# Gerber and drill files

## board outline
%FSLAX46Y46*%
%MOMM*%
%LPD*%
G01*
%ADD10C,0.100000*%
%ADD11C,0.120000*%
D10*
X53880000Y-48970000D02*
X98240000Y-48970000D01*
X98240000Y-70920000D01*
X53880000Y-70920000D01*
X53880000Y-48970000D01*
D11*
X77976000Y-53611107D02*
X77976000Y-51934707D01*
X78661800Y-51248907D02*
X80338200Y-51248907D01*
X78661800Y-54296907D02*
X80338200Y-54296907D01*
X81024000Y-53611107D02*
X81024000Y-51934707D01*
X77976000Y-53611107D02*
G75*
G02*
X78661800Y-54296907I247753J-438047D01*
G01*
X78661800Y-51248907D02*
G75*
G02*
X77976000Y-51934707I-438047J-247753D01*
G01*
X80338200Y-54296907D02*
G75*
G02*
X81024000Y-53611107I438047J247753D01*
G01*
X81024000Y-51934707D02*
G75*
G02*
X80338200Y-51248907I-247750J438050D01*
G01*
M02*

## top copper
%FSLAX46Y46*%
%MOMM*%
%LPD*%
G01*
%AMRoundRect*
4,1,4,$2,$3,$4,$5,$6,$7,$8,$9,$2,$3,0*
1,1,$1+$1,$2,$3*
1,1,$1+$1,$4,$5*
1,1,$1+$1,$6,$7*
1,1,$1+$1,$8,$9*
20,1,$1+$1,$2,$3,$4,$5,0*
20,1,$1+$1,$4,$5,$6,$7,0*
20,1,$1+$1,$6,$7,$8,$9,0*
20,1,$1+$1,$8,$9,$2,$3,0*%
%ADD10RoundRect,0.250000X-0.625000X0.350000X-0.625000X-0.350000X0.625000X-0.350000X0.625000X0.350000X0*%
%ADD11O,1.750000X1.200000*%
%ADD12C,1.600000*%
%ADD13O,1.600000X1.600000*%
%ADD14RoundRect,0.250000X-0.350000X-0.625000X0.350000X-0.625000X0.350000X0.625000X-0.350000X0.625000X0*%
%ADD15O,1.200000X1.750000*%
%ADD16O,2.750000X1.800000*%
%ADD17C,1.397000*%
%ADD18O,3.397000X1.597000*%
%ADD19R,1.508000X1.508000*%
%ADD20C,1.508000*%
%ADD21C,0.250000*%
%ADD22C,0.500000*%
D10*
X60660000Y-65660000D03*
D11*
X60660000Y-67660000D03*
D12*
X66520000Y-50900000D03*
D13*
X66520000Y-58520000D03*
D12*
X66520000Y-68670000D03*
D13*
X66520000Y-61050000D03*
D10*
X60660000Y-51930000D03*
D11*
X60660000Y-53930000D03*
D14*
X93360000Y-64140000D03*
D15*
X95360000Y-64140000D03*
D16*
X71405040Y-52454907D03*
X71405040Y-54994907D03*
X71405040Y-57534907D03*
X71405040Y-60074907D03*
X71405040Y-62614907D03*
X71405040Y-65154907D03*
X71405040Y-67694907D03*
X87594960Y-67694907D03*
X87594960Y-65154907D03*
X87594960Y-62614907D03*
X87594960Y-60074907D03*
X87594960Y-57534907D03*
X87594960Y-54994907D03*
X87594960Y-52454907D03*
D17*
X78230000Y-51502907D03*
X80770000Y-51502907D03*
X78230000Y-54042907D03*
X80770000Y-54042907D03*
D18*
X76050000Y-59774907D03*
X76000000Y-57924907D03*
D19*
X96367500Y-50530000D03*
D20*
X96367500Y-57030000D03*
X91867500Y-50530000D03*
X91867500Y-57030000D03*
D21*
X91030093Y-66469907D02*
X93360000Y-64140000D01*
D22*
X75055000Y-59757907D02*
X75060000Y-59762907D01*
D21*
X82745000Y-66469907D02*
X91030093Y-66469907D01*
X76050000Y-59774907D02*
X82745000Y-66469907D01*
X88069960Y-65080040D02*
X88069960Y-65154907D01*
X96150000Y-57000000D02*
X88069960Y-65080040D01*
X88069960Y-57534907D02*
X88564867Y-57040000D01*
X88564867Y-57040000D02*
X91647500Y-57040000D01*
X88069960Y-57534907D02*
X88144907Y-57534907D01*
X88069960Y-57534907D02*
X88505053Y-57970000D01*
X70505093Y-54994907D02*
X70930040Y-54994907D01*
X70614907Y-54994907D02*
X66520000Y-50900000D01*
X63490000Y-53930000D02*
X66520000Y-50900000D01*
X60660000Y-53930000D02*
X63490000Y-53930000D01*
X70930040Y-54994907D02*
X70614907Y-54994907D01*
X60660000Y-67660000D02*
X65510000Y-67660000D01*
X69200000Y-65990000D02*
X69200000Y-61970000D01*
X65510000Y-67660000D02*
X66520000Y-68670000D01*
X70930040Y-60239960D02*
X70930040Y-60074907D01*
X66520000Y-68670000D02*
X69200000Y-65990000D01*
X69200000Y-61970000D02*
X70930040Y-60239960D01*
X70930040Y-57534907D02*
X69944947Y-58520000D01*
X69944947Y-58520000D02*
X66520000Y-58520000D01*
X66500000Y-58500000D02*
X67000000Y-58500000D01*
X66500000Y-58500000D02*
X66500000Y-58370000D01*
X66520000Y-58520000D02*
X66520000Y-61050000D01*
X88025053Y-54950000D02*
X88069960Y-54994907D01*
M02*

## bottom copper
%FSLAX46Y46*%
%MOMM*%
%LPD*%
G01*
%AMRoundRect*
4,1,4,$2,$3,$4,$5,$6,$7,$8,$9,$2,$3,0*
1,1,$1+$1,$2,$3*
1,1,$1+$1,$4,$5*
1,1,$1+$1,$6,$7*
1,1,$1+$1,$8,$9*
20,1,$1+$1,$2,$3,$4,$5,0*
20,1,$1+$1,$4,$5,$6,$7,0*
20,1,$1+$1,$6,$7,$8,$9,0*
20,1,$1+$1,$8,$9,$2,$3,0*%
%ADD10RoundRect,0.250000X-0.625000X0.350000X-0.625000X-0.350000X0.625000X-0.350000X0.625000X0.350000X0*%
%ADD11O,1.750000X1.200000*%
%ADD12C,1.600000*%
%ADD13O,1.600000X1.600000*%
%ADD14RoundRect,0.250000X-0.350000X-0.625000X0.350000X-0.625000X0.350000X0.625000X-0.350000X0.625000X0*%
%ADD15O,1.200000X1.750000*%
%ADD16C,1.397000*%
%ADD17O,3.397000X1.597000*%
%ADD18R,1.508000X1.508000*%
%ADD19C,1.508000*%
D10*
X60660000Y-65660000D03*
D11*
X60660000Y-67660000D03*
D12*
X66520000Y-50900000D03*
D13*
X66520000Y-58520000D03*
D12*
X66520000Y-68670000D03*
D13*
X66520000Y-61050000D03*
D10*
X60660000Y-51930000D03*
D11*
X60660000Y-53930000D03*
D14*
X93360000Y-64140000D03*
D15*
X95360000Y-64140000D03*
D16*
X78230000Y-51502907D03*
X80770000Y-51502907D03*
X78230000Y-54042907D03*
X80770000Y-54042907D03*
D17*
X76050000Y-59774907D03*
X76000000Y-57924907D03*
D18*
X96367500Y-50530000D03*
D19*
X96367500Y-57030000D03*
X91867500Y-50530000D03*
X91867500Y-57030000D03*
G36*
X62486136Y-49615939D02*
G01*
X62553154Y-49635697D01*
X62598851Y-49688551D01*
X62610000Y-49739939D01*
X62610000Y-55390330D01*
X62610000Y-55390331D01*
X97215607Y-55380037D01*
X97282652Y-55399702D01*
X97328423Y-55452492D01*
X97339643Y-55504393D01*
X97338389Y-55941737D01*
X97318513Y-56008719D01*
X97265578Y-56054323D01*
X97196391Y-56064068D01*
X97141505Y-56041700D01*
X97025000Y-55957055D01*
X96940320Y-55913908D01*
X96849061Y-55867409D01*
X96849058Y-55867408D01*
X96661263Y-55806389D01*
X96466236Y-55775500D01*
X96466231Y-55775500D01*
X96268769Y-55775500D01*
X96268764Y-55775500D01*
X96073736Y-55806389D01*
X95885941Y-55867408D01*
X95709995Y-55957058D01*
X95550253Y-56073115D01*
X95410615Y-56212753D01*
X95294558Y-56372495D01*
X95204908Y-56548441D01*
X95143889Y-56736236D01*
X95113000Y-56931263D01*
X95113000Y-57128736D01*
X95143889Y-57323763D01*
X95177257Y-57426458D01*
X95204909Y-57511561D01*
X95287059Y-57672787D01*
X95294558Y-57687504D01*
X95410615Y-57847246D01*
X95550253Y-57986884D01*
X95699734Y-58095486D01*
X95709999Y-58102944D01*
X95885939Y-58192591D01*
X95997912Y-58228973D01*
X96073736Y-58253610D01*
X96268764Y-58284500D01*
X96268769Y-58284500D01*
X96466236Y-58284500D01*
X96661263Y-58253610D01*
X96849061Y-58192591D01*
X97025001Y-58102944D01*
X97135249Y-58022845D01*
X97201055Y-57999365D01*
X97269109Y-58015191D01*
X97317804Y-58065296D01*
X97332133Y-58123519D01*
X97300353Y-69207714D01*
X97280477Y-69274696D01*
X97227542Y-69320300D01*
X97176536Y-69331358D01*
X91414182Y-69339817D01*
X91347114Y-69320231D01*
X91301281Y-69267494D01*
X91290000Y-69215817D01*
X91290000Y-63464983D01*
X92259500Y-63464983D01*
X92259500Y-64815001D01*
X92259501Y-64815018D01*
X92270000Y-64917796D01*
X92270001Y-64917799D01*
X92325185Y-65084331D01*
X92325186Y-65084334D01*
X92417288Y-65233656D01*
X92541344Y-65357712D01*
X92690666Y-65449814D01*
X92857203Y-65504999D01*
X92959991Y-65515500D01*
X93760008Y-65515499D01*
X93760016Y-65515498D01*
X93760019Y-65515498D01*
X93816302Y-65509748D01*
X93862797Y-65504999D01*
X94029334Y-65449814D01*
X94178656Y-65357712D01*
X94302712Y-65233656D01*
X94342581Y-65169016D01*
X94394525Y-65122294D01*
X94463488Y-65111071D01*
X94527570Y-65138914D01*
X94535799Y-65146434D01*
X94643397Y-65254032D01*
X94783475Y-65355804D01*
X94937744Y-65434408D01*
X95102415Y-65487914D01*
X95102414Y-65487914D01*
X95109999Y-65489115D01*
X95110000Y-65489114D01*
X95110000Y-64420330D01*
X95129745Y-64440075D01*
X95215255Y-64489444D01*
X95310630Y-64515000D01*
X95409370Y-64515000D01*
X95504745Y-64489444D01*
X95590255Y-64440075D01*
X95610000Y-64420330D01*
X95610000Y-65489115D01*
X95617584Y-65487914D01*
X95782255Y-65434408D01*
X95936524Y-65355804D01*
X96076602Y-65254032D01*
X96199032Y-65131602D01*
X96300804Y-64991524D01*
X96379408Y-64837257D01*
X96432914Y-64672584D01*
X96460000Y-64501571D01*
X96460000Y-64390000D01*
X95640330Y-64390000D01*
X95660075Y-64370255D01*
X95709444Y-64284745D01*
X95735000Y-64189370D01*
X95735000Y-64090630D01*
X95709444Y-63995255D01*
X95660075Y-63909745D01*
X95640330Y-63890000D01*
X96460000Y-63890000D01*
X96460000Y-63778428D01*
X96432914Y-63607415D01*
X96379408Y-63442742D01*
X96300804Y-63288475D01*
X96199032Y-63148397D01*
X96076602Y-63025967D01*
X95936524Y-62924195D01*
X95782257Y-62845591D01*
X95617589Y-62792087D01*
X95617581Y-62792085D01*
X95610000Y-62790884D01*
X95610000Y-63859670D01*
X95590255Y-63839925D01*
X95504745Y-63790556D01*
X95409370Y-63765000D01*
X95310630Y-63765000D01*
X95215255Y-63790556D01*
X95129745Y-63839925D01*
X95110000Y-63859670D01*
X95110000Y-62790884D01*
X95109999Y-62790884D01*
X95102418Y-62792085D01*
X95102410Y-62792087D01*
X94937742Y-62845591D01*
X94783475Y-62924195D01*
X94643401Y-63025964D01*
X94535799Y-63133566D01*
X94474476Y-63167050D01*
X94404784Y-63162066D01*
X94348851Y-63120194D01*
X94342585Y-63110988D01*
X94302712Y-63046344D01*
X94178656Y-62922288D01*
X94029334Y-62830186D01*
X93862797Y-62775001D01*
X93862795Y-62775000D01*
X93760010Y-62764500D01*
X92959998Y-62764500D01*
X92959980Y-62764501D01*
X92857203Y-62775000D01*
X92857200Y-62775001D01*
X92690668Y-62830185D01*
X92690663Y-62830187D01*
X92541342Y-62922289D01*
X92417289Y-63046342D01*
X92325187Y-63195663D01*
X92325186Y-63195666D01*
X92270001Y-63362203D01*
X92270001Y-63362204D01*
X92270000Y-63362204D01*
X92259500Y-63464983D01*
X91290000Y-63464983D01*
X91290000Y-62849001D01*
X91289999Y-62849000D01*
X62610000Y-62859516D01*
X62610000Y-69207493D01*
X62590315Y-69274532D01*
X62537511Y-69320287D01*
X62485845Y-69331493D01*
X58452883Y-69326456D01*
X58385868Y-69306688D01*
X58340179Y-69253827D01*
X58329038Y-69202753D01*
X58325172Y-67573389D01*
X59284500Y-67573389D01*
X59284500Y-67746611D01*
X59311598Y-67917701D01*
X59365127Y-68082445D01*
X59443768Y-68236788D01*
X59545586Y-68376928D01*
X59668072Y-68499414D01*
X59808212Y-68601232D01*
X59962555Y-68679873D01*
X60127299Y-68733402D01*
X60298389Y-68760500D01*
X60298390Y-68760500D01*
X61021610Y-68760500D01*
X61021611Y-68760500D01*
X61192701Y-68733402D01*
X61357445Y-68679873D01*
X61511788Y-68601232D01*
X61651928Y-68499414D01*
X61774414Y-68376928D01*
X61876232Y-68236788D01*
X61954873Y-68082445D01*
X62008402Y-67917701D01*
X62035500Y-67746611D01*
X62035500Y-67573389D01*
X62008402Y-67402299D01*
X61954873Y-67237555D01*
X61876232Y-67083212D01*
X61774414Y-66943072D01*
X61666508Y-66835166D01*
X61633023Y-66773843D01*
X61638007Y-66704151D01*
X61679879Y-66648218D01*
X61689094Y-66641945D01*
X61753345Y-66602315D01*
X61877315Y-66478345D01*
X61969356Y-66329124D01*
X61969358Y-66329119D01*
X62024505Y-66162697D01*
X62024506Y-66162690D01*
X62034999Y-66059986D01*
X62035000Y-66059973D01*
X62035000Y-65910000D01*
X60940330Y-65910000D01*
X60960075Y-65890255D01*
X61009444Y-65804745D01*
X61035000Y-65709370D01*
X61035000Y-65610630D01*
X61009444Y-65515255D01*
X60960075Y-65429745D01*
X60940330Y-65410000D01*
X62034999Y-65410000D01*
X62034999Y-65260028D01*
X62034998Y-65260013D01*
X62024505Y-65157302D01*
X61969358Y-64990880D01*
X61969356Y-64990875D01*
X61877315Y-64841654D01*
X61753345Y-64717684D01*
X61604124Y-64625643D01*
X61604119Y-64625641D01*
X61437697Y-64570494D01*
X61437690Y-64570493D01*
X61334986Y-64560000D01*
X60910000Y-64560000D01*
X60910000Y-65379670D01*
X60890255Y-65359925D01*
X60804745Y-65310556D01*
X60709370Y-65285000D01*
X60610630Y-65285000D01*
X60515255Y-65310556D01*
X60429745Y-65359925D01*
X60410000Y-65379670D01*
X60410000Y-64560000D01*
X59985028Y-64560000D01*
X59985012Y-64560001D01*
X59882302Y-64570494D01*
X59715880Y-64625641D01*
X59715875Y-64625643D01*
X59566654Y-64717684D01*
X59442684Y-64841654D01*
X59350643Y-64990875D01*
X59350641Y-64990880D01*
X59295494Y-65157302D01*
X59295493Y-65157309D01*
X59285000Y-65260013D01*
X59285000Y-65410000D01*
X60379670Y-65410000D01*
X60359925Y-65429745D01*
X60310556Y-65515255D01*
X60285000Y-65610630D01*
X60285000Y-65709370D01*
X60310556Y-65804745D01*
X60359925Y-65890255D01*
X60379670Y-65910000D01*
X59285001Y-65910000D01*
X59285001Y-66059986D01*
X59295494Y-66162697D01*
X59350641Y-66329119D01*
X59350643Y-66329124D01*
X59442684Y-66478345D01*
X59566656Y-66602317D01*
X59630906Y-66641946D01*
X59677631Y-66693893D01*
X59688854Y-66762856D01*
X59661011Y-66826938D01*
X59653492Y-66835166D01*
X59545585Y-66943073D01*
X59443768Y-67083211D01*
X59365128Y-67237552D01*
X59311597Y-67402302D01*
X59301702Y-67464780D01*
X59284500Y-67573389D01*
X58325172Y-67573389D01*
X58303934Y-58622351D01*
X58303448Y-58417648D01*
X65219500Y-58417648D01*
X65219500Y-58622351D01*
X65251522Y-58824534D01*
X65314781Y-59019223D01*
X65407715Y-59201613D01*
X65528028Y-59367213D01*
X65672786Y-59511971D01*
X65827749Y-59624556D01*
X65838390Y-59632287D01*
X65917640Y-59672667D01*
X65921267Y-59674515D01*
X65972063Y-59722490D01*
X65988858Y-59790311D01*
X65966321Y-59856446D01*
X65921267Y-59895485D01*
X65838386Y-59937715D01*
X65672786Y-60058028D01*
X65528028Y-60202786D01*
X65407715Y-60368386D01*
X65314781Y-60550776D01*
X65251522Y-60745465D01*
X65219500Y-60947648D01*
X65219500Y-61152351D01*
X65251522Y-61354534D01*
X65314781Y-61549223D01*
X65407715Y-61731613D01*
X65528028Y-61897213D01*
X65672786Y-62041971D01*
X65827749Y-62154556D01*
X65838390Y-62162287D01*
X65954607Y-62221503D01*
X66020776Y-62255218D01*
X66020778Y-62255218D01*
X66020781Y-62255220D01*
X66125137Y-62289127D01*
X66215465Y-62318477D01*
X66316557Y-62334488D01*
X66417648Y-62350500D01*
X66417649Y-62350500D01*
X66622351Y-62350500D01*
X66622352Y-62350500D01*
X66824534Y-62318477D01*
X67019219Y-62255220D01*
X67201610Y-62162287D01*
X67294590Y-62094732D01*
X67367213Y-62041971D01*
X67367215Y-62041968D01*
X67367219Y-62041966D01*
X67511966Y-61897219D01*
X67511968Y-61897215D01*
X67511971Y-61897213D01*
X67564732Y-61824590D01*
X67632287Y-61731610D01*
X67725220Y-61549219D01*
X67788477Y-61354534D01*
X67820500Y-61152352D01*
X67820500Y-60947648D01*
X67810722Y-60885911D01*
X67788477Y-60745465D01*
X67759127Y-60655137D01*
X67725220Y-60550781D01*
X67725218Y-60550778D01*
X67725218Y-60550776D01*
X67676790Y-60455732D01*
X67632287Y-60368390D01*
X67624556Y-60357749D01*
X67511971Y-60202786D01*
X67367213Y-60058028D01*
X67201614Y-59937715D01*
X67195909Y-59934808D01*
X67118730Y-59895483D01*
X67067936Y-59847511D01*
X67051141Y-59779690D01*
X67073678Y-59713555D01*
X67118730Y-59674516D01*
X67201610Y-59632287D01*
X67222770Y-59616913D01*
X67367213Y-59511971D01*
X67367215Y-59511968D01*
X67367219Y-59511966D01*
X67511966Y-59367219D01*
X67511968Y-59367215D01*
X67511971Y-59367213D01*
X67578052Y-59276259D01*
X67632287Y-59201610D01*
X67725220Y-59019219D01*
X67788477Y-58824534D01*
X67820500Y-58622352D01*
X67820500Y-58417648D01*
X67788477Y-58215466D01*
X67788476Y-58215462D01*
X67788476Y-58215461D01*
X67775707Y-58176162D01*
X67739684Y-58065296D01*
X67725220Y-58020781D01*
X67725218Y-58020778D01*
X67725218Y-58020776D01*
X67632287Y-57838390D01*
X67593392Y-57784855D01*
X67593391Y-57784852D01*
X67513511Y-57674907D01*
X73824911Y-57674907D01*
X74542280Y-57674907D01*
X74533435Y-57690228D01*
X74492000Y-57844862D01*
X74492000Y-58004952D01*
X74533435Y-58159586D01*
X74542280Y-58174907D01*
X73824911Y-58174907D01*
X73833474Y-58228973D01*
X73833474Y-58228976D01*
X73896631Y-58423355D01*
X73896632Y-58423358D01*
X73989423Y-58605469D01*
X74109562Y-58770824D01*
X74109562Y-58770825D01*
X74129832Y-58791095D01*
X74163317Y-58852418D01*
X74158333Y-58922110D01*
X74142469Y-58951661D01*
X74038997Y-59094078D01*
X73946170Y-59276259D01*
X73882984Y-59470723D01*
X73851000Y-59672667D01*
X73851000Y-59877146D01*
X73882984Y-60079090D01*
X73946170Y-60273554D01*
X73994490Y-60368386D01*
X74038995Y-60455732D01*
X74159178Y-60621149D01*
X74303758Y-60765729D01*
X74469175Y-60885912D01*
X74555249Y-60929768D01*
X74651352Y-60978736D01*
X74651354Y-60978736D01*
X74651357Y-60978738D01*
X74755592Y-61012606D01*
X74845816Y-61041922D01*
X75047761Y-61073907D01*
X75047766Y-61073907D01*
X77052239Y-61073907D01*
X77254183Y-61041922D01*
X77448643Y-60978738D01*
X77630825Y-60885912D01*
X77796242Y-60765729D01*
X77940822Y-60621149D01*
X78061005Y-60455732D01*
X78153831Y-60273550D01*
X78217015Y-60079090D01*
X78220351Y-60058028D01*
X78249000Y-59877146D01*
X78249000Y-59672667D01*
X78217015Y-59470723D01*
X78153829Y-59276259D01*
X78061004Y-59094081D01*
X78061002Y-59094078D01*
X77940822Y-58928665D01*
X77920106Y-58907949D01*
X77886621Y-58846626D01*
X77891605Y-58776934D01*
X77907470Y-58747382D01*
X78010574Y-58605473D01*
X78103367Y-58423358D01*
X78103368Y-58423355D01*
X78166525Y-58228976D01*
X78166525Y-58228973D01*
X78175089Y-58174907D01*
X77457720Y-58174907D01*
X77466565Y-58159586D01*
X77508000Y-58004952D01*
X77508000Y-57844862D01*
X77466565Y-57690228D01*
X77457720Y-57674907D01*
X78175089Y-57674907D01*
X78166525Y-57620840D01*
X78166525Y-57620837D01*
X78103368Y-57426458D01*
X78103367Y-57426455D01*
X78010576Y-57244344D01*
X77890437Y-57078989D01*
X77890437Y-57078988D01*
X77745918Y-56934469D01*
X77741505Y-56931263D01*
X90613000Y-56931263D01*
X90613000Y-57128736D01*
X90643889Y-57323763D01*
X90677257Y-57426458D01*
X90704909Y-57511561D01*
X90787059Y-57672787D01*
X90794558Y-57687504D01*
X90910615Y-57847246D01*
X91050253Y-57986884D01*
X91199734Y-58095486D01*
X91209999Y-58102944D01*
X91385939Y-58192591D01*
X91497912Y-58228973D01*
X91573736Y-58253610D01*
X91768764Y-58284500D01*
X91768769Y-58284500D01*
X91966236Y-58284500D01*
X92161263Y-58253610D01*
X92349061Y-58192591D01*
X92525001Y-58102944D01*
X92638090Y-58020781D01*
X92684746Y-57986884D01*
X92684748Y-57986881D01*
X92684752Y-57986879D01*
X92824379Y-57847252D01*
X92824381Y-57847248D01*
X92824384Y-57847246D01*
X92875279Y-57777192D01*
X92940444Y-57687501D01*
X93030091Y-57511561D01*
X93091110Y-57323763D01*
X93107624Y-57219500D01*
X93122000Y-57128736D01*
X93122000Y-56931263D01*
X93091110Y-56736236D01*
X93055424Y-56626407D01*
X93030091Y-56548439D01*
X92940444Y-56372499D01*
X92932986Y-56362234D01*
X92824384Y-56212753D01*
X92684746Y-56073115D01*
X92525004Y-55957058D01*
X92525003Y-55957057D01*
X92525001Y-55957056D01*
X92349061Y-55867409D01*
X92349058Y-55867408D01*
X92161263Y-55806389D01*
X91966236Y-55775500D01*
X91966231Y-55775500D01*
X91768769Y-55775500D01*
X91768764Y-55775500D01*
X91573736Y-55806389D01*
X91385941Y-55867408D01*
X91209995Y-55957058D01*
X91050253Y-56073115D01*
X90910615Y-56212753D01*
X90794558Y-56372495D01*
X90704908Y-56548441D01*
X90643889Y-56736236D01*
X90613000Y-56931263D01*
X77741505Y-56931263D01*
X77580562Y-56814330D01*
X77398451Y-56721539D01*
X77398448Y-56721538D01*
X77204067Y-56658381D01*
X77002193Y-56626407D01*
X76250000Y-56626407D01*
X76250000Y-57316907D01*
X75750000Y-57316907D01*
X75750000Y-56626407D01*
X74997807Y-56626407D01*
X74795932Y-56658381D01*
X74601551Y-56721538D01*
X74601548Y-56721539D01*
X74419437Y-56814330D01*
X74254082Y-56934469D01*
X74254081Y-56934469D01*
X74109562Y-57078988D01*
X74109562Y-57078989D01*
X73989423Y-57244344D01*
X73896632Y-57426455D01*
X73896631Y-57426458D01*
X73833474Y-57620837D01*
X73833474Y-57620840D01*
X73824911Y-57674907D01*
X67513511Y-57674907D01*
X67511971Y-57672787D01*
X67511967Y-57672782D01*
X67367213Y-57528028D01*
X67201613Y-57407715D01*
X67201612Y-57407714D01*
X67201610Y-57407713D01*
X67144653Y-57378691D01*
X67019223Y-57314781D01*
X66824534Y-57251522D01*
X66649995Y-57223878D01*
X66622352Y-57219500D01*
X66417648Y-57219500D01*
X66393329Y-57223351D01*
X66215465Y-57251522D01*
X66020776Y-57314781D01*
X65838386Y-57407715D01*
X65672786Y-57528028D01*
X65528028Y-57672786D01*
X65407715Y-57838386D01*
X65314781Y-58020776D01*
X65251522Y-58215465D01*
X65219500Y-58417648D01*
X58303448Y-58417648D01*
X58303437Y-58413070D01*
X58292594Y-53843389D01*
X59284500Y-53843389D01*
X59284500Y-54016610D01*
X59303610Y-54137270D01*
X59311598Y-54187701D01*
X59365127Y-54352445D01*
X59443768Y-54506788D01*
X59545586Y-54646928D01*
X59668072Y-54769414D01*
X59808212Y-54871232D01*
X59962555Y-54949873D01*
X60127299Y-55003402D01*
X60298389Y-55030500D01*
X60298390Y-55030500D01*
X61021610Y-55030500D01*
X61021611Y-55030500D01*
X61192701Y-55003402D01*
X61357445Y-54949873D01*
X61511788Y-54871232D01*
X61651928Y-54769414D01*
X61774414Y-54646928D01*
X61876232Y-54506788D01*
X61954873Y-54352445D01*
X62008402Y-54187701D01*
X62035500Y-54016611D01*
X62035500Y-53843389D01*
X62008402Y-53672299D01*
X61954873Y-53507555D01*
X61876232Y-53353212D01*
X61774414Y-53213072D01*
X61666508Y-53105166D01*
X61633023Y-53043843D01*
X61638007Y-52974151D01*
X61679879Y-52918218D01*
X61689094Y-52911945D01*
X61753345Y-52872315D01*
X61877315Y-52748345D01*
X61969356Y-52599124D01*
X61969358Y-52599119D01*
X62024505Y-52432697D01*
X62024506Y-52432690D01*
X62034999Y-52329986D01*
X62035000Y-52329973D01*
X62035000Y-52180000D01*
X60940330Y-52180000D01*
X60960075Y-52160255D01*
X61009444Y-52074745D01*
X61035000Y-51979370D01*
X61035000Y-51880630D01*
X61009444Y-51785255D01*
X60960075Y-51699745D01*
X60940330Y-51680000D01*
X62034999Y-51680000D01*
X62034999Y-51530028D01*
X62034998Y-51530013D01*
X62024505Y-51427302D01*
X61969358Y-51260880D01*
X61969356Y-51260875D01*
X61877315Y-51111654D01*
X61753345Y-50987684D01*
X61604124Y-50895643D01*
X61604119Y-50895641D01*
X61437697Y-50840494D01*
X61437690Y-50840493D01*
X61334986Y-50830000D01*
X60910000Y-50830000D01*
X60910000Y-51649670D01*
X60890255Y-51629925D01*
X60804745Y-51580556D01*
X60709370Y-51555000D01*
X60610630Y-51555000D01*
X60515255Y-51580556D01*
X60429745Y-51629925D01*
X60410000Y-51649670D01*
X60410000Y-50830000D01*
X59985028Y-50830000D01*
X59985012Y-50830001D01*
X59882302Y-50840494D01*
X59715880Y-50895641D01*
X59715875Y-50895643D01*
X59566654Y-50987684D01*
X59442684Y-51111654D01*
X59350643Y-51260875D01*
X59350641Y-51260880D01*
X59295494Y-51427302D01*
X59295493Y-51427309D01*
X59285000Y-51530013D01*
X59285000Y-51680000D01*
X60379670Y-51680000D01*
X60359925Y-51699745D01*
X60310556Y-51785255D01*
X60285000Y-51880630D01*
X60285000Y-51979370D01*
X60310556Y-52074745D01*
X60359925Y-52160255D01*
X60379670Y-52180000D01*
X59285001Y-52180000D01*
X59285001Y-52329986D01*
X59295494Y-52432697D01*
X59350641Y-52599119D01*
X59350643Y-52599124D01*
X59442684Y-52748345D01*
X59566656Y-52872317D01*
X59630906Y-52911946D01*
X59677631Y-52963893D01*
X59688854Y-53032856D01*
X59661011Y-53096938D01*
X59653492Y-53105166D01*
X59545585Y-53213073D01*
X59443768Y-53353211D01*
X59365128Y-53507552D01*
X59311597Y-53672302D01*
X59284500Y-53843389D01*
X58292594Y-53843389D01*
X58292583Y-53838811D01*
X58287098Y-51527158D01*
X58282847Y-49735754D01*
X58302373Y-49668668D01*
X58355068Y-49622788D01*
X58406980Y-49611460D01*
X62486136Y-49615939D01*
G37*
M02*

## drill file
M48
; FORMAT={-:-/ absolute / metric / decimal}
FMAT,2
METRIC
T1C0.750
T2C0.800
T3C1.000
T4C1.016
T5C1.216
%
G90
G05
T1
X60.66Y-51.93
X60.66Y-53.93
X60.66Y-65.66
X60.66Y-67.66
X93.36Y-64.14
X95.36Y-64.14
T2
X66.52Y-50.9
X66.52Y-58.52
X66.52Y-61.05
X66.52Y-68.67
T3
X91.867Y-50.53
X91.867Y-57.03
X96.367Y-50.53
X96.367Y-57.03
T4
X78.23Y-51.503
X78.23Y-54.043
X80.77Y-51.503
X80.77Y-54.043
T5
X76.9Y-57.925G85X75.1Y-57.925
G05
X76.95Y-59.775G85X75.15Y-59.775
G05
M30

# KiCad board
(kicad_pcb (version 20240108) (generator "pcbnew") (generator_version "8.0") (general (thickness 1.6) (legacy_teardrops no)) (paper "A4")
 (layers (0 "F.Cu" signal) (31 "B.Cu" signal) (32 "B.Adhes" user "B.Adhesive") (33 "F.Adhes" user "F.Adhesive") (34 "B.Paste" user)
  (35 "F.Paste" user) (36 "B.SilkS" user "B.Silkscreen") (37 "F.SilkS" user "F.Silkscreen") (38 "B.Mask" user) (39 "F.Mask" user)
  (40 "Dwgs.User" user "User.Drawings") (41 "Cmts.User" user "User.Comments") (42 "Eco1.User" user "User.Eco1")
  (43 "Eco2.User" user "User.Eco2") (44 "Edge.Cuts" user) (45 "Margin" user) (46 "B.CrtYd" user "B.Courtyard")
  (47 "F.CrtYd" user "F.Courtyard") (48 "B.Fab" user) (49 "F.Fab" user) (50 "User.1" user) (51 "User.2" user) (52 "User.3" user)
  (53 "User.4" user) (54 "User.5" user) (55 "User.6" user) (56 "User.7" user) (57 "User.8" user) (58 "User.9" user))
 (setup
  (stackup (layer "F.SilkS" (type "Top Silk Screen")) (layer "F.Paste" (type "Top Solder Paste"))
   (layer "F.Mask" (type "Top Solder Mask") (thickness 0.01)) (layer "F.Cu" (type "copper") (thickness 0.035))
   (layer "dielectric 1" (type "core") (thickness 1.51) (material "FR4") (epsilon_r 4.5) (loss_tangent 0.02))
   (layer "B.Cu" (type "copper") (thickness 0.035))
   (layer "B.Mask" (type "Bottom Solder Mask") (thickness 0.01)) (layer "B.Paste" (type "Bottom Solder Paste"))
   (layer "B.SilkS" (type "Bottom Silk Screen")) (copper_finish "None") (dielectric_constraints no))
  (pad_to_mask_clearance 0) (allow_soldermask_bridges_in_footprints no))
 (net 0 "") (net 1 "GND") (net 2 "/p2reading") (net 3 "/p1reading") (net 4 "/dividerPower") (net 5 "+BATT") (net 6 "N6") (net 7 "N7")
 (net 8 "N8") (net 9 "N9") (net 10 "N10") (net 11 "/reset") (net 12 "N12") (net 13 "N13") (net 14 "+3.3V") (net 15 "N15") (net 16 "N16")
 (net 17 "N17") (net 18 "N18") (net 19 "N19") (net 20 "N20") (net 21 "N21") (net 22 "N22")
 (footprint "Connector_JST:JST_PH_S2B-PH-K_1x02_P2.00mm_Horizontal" (layer "F.Cu") (at 60.66 65.66 -90)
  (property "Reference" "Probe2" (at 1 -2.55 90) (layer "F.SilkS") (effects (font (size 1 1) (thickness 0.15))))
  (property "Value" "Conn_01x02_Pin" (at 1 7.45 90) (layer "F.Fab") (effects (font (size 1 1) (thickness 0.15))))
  (pad "1" thru_hole roundrect (at 0 0 270) (size 1.2 1.75) (drill 0.75) (layers "*.Cu" "*.Mask") (remove_unused_layers no)
   (roundrect_rratio 0.208333) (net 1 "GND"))
  (pad "2" thru_hole oval (at 2 0 270) (size 1.2 1.75) (drill 0.75) (layers "*.Cu" "*.Mask") (remove_unused_layers no) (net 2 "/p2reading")))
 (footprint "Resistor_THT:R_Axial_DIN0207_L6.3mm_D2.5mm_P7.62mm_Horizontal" (layer "F.Cu") (at 66.52 50.9 -90)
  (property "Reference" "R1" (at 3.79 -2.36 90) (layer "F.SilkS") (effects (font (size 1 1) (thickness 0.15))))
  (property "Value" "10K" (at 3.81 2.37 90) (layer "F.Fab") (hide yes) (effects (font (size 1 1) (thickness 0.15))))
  (pad "1" thru_hole circle (at 0 0 270) (size 1.6 1.6) (drill 0.8) (layers "*.Cu" "*.Mask") (remove_unused_layers no) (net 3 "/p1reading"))
  (pad "2" thru_hole oval (at 7.62 0 270) (size 1.6 1.6) (drill 0.8) (layers "*.Cu" "*.Mask") (remove_unused_layers no)
   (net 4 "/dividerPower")))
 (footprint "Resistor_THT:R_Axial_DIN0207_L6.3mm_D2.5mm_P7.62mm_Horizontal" (layer "F.Cu") (at 66.52 68.67 90)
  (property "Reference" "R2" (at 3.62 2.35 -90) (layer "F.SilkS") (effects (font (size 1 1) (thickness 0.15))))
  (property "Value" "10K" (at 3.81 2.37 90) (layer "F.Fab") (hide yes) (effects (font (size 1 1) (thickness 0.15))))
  (pad "1" thru_hole circle (at 0 0 90) (size 1.6 1.6) (drill 0.8) (layers "*.Cu" "*.Mask") (remove_unused_layers no) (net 2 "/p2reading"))
  (pad "2" thru_hole oval (at 7.62 0 90) (size 1.6 1.6) (drill 0.8) (layers "*.Cu" "*.Mask") (remove_unused_layers no)
   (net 4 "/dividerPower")))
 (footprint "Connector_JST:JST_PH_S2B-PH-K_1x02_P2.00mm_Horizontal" (layer "F.Cu") (at 60.66 51.93 -90)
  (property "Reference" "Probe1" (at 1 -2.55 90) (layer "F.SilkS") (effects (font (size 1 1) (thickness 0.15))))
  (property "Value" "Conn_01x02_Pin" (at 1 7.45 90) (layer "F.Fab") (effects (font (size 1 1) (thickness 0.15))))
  (pad "1" thru_hole roundrect (at 0 0 270) (size 1.2 1.75) (drill 0.75) (layers "*.Cu" "*.Mask") (remove_unused_layers no)
   (roundrect_rratio 0.208333) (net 1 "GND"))
  (pad "2" thru_hole oval (at 2 0 270) (size 1.2 1.75) (drill 0.75) (layers "*.Cu" "*.Mask") (remove_unused_layers no) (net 3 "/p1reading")))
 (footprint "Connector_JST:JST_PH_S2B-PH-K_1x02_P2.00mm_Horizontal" (layer "F.Cu") (at 93.36 64.14)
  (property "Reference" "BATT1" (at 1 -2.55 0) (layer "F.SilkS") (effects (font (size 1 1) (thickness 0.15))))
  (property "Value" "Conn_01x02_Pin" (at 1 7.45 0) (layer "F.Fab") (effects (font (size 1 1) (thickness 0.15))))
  (pad "1" thru_hole roundrect (at 0 0) (size 1.2 1.75) (drill 0.75) (layers "*.Cu" "*.Mask") (remove_unused_layers no)
   (roundrect_rratio 0.208333) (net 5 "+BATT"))
  (pad "2" thru_hole oval (at 2 0) (size 1.2 1.75) (drill 0.75) (layers "*.Cu" "*.Mask") (remove_unused_layers no) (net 1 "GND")))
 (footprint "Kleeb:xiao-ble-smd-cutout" (layer "F.Cu") (at 79.5 60.074907)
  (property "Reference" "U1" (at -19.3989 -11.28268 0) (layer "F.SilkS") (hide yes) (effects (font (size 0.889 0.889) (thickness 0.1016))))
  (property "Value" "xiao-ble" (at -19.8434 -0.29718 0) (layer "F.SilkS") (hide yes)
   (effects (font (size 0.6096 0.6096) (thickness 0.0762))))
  (fp_line (start -1.524 -6.4638) (end -1.524 -8.1402) (stroke (width 0.12) (type solid)) (layer "Edge.Cuts"))
  (fp_line (start -0.8382 -8.826) (end 0.8382 -8.826) (stroke (width 0.12) (type solid)) (layer "Edge.Cuts"))
  (fp_line (start -0.8382 -5.778) (end 0.8382 -5.778) (stroke (width 0.12) (type solid)) (layer "Edge.Cuts"))
  (fp_line (start 1.524 -6.4638) (end 1.524 -8.1402) (stroke (width 0.12) (type solid)) (layer "Edge.Cuts"))
  (fp_arc (start -1.524 -6.4638) (mid -0.920391 -6.381609) (end -0.8382 -5.778) (stroke (width 0.12) (type solid)) (layer "Edge.Cuts"))
  (fp_arc (start -0.8382 -8.826) (mid -0.920391 -8.222391) (end -1.524 -8.1402) (stroke (width 0.12) (type solid)) (layer "Edge.Cuts"))
  (fp_arc (start 0.8382 -5.778) (mid 0.920391 -6.381609) (end 1.524 -6.4638) (stroke (width 0.12) (type solid)) (layer "Edge.Cuts"))
  (fp_arc (start 1.524 -8.1402) (mid 0.920393 -8.222393) (end 0.8382 -8.826) (stroke (width 0.12) (type solid)) (layer "Edge.Cuts"))
  (pad "1" smd oval (at -8.56996 -7.62 180) (size 2.75 1.8) (drill (offset -0.475 0)) (layers "F.Cu" "F.Paste" "F.Mask") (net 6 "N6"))
  (pad "2" smd oval (at -8.56996 -5.08 180) (size 2.75 1.8) (drill (offset -0.475 0)) (layers "F.Cu" "F.Paste" "F.Mask")
   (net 3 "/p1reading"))
  (pad "3" smd oval (at -8.56996 -2.54 180) (size 2.75 1.8) (drill (offset -0.475 0)) (layers "F.Cu" "F.Paste" "F.Mask")
   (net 4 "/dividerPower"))
  (pad "4" smd oval (at -8.56996 0 180) (size 2.75 1.8) (drill (offset -0.475 0)) (layers "F.Cu" "F.Paste" "F.Mask") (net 2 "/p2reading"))
  (pad "5" smd oval (at -8.56996 2.54 180) (size 2.75 1.8) (drill (offset -0.475 0)) (layers "F.Cu" "F.Paste" "F.Mask") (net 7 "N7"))
  (pad "6" smd oval (at -8.56996 5.08 180) (size 2.75 1.8) (drill (offset -0.475 0)) (layers "F.Cu" "F.Paste" "F.Mask") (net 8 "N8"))
  (pad "7" smd oval (at -8.56996 7.62 180) (size 2.75 1.8) (drill (offset -0.475 0)) (layers "F.Cu" "F.Paste" "F.Mask") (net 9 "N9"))
  (pad "8" smd oval (at 8.56996 7.62) (size 2.75 1.8) (drill (offset -0.475 0)) (layers "F.Cu" "F.Paste" "F.Mask") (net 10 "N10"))
  (pad "9" smd oval (at 8.56996 5.08) (size 2.75 1.8) (drill (offset -0.475 0)) (layers "F.Cu" "F.Paste" "F.Mask") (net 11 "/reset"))
  (pad "10" smd oval (at 8.56996 2.54) (size 2.75 1.8) (drill (offset -0.475 0)) (layers "F.Cu" "F.Paste" "F.Mask") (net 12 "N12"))
  (pad "11" smd oval (at 8.56996 0) (size 2.75 1.8) (drill (offset -0.475 0)) (layers "F.Cu" "F.Paste" "F.Mask") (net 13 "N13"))
  (pad "12" smd oval (at 8.56996 -2.54) (size 2.75 1.8) (drill (offset -0.475 0)) (layers "F.Cu" "F.Paste" "F.Mask") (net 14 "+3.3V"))
  (pad "13" smd oval (at 8.56996 -5.08) (size 2.75 1.8) (drill (offset -0.475 0)) (layers "F.Cu" "F.Paste" "F.Mask") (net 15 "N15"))
  (pad "14" smd oval (at 8.56996 -7.62) (size 2.75 1.8) (drill (offset -0.475 0)) (layers "F.Cu" "F.Paste" "F.Mask") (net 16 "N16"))
  (pad "15" thru_hole circle (at -1.27 -8.572 90) (size 1.397 1.397) (drill 1.016) (layers "*.Cu" "*.Mask") (remove_unused_layers no)
   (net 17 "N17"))
  (pad "16" thru_hole circle (at 1.27 -8.572 90) (size 1.397 1.397) (drill 1.016) (layers "*.Cu" "*.Mask") (remove_unused_layers no)
   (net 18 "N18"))
  (pad "17" thru_hole circle (at -1.27 -6.032 90) (size 1.397 1.397) (drill 1.016) (layers "*.Cu" "*.Mask") (remove_unused_layers no)
   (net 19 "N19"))
  (pad "18" thru_hole circle (at 1.27 -6.032 90) (size 1.397 1.397) (drill 1.016) (layers "*.Cu" "*.Mask") (remove_unused_layers no)
   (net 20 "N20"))
  (pad "19" thru_hole oval (at -3.45 -0.3 180) (size 3.397 1.597) (drill oval 3.016 1.216) (layers "*.Cu" "*.Mask")
   (remove_unused_layers no) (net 5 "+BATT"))
  (pad "20" thru_hole oval (at -3.5 -2.15 180) (size 3.397 1.597) (drill oval 3.016 1.216) (layers "*.Cu" "*.Mask")
   (remove_unused_layers no) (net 1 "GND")))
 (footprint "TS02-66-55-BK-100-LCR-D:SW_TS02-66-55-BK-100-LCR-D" (layer "F.Cu") (at 94.1175 53.78 -90)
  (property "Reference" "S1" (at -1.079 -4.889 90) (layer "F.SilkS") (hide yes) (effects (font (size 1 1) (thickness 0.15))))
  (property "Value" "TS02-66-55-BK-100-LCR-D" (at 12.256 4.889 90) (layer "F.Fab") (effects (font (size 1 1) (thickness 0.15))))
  (pad "1" thru_hole rect (at -3.25 -2.25 270) (size 1.508 1.508) (drill 1) (layers "*.Cu" "*.Mask") (remove_unused_layers no)
   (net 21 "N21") (solder_mask_margin 0.102))
  (pad "2" thru_hole circle (at 3.25 -2.25 270) (size 1.508 1.508) (drill 1) (layers "*.Cu" "*.Mask") (remove_unused_layers no)
   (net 11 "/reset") (solder_mask_margin 0.102))
  (pad "3" thru_hole circle (at -3.25 2.25 270) (size 1.508 1.508) (drill 1) (layers "*.Cu" "*.Mask") (remove_unused_layers no)
   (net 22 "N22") (solder_mask_margin 0.102))
  (pad "4" thru_hole circle (at 3.25 2.25 270) (size 1.508 1.508) (drill 1) (layers "*.Cu" "*.Mask") (remove_unused_layers no)
   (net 14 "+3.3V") (solder_mask_margin 0.102)))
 (gr_rect (start 53.88 48.97) (end 98.24 70.92) (stroke (width 0.1) (type default)) (fill none) (layer "Edge.Cuts"))
 (segment (start 91.030093 66.469907) (end 93.36 64.14) (width 0.25) (layer "F.Cu") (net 5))
 (segment (start 75.055 59.757907) (end 75.06 59.762907) (width 0.5) (layer "F.Cu") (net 5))
 (segment (start 82.745 66.469907) (end 91.030093 66.469907) (width 0.25) (layer "F.Cu") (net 5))
 (segment (start 76.05 59.774907) (end 82.745 66.469907) (width 0.25) (layer "F.Cu") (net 5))
 (segment (start 88.06996 65.08004) (end 88.06996 65.154907) (width 0.25) (layer "F.Cu") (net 11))
 (segment (start 96.15 57) (end 88.06996 65.08004) (width 0.25) (layer "F.Cu") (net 11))
 (segment (start 88.06996 57.534907) (end 88.564867 57.04) (width 0.25) (layer "F.Cu") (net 14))
 (segment (start 88.564867 57.04) (end 91.6475 57.04) (width 0.25) (layer "F.Cu") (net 14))
 (segment (start 88.06996 57.534907) (end 88.144907 57.534907) (width 0.25) (layer "F.Cu") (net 14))
 (segment (start 88.06996 57.534907) (end 88.505053 57.97) (width 0.25) (layer "F.Cu") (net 14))
 (segment (start 70.505093 54.994907) (end 70.93004 54.994907) (width 0.25) (layer "F.Cu") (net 3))
 (segment (start 70.614907 54.994907) (end 66.52 50.9) (width 0.25) (layer "F.Cu") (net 3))
 (segment (start 63.49 53.93) (end 66.52 50.9) (width 0.25) (layer "F.Cu") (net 3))
 (segment (start 60.66 53.93) (end 63.49 53.93) (width 0.25) (layer "F.Cu") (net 3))
 (segment (start 70.93004 54.994907) (end 70.614907 54.994907) (width 0.25) (layer "F.Cu") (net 3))
 (segment (start 60.66 67.66) (end 65.51 67.66) (width 0.25) (layer "F.Cu") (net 2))
 (segment (start 69.2 65.99) (end 69.2 61.97) (width 0.25) (layer "F.Cu") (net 2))
 (segment (start 65.51 67.66) (end 66.52 68.67) (width 0.25) (layer "F.Cu") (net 2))
 (segment (start 70.93004 60.23996) (end 70.93004 60.074907) (width 0.25) (layer "F.Cu") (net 2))
 (segment (start 66.52 68.67) (end 69.2 65.99) (width 0.25) (layer "F.Cu") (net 2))
 (segment (start 69.2 61.97) (end 70.93004 60.23996) (width 0.25) (layer "F.Cu") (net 2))
 (segment (start 70.93004 57.534907) (end 69.944947 58.52) (width 0.25) (layer "F.Cu") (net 4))
 (segment (start 69.944947 58.52) (end 66.52 58.52) (width 0.25) (layer "F.Cu") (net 4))
 (segment (start 66.5 58.5) (end 67 58.5) (width 0.25) (layer "F.Cu") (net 4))
 (segment (start 66.5 58.5) (end 66.5 58.37) (width 0.25) (layer "F.Cu") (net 4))
 (segment (start 66.52 58.52) (end 66.52 61.05) (width 0.25) (layer "F.Cu") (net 4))
 (segment (start 88.025053 54.95) (end 88.06996 54.994907) (width 0.25) (layer "F.Cu") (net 15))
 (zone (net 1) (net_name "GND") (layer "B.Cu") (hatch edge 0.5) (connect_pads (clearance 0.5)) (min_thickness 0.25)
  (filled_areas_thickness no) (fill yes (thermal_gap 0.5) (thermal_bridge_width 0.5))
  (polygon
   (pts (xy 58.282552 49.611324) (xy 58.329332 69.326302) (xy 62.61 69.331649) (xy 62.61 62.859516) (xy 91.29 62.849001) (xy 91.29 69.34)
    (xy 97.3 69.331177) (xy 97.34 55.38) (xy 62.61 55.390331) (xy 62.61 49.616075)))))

